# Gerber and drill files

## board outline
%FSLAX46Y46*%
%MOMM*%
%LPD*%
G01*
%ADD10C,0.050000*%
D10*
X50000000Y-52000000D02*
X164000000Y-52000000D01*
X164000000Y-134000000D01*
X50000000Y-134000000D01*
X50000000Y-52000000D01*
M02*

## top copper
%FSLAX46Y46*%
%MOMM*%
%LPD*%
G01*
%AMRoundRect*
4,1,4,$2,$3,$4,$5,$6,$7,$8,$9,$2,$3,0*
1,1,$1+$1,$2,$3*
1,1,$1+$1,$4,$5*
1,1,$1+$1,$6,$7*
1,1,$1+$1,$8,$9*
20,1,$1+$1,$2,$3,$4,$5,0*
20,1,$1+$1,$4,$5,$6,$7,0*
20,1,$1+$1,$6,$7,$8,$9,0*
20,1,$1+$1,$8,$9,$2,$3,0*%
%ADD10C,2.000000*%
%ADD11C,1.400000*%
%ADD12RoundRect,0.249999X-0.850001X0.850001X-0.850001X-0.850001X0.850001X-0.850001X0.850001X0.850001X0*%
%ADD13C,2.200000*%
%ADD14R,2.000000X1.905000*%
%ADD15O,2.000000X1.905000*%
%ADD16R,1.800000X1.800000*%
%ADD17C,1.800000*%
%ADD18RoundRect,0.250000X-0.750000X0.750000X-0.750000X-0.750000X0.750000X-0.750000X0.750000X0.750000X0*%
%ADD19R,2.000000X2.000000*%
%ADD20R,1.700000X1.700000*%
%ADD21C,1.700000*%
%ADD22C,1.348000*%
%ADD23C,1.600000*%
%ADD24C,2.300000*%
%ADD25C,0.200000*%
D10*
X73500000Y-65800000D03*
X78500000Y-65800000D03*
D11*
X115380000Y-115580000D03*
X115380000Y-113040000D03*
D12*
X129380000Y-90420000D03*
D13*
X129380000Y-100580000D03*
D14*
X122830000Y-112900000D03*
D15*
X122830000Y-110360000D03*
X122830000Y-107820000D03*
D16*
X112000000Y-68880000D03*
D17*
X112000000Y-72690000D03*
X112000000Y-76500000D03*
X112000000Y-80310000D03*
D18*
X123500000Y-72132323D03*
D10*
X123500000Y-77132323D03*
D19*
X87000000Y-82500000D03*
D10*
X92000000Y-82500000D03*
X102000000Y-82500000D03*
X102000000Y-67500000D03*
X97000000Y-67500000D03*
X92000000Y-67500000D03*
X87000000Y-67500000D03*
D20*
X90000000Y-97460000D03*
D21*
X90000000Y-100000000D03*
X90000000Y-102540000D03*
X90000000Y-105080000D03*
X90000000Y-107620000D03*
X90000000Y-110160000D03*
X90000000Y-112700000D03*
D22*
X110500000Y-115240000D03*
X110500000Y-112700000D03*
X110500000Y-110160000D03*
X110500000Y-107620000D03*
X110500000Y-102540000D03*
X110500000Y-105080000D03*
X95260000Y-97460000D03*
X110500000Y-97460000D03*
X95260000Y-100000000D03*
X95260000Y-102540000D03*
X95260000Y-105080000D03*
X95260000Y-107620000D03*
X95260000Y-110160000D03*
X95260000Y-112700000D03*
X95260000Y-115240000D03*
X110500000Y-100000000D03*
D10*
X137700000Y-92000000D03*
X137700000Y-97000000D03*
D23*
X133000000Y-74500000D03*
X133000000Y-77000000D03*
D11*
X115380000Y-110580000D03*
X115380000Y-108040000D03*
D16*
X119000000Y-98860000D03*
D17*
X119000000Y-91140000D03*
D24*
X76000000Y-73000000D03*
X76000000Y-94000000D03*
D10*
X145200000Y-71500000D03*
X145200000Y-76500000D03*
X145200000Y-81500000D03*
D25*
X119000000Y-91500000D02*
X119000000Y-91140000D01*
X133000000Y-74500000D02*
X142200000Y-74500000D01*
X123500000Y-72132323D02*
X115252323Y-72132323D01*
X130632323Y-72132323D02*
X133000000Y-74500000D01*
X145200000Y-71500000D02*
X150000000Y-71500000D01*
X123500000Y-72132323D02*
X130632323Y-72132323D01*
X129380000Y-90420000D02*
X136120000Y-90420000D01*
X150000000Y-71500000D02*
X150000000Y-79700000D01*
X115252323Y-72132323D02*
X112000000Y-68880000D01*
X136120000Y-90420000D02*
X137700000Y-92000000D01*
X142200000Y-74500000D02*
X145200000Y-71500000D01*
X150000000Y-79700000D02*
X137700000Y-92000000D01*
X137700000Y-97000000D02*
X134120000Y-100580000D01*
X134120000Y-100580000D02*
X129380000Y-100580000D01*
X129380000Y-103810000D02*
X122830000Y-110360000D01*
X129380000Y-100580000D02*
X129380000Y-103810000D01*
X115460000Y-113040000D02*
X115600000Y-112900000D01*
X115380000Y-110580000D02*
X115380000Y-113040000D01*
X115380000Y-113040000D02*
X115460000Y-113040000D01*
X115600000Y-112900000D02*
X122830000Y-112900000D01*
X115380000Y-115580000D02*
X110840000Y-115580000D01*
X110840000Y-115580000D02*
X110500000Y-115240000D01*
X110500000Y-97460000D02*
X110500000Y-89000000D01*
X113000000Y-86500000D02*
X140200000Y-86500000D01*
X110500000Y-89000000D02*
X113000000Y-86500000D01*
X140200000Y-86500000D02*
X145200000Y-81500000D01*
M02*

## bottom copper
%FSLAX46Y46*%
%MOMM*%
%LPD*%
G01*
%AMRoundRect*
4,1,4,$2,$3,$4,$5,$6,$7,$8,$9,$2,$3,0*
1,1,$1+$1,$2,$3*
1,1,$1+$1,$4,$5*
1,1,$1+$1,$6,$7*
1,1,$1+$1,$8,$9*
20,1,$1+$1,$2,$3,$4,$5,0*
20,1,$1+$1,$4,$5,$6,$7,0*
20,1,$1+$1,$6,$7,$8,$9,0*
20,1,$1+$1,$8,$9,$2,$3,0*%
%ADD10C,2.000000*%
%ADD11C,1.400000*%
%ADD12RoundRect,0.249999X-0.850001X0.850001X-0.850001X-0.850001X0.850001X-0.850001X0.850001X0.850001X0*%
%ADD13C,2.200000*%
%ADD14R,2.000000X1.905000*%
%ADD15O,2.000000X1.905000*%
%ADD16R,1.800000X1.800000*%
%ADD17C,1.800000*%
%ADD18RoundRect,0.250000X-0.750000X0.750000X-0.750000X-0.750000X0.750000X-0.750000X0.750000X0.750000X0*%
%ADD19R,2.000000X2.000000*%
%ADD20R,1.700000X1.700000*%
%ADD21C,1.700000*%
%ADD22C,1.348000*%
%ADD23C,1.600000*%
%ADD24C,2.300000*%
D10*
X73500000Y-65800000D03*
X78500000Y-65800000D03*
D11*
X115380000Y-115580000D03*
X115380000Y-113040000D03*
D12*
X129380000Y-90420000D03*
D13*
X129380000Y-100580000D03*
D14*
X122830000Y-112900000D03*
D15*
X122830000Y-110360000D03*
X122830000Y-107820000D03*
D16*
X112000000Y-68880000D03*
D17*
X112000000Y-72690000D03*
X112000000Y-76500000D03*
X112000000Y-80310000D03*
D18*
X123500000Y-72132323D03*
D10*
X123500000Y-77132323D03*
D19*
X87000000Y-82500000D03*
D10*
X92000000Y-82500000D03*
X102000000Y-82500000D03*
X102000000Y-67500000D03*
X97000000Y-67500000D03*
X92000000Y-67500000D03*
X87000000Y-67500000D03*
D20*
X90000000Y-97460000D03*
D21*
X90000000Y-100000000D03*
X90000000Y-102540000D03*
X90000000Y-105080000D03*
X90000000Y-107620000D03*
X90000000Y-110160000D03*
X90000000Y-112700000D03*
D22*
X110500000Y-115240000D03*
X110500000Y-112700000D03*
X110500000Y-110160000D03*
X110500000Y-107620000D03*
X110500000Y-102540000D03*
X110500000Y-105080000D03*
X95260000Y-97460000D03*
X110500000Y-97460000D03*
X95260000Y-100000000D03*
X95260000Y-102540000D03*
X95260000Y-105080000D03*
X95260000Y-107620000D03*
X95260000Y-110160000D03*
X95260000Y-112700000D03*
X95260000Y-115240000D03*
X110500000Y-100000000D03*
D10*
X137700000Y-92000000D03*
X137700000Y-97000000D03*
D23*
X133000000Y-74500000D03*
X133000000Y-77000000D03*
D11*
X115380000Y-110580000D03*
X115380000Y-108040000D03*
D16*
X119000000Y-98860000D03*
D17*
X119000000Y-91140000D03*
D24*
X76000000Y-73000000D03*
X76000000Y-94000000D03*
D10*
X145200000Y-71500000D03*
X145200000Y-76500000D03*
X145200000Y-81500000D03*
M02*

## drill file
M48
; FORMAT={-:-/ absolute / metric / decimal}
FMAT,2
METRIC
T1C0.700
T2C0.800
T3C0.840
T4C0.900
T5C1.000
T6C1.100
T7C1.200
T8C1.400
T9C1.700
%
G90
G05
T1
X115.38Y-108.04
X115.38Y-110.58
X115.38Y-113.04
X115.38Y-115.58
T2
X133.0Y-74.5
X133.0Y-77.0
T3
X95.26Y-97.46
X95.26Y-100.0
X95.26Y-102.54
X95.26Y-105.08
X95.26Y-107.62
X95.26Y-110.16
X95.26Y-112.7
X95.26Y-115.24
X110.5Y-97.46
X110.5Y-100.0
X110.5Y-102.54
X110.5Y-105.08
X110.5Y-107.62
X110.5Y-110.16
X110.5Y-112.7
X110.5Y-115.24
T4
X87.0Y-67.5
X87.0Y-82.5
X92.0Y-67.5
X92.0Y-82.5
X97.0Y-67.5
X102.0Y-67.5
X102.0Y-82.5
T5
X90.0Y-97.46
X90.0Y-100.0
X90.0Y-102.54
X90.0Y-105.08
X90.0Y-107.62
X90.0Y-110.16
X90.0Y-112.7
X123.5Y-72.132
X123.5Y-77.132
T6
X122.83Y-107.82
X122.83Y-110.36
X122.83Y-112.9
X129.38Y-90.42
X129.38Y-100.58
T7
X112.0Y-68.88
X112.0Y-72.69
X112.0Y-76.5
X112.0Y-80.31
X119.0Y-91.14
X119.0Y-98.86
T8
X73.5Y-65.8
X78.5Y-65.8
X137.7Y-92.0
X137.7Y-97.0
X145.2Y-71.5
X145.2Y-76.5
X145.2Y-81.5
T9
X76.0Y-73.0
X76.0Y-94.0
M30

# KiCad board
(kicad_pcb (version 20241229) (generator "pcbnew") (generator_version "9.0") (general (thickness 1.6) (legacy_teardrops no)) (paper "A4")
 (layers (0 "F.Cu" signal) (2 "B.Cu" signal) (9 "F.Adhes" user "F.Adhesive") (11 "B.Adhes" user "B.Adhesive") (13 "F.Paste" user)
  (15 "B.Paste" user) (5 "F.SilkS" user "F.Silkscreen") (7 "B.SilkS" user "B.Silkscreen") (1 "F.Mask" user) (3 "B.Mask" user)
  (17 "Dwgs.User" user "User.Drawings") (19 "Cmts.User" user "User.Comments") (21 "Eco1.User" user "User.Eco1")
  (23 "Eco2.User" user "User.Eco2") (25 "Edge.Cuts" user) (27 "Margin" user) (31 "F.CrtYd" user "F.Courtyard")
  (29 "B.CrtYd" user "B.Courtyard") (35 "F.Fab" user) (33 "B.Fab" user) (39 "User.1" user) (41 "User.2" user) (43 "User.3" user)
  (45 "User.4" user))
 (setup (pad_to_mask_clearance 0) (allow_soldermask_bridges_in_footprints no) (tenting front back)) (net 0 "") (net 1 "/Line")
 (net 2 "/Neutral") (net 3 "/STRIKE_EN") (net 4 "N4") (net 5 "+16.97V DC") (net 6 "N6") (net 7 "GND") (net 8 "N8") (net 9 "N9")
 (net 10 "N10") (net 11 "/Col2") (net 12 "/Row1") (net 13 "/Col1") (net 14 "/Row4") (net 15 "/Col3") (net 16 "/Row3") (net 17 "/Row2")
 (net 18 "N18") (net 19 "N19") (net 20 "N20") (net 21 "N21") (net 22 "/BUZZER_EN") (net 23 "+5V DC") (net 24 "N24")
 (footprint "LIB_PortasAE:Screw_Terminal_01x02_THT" (layer "F.Cu") (at 73.5 65.8)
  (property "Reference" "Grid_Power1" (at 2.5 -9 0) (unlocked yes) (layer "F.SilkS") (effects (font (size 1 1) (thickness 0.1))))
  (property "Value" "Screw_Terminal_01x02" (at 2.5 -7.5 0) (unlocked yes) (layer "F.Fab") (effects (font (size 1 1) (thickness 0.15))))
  (pad "1" thru_hole circle (at 0 0) (size 2 2) (drill 1.4) (layers "*.Cu" "*.Mask") (remove_unused_layers no) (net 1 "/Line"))
  (pad "2" thru_hole circle (at 5 0) (size 2 2) (drill 1.4) (layers "*.Cu" "*.Mask") (remove_unused_layers no) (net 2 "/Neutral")))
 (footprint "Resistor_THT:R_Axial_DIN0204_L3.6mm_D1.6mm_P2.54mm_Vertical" (layer "F.Cu") (at 115.38 115.58 90)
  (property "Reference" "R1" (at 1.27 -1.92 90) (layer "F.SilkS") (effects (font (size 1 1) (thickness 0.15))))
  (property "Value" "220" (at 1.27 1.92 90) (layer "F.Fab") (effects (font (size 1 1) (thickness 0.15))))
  (pad "1" thru_hole circle (at 0 0 90) (size 1.4 1.4) (drill 0.7) (layers "*.Cu" "*.Mask") (remove_unused_layers no) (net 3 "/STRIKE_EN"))
  (pad "2" thru_hole circle (at 2.54 0 90) (size 1.4 1.4) (drill 0.7) (layers "*.Cu" "*.Mask") (remove_unused_layers no) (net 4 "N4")))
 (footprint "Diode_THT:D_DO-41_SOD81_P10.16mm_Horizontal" (layer "F.Cu") (at 129.38 90.42 -90)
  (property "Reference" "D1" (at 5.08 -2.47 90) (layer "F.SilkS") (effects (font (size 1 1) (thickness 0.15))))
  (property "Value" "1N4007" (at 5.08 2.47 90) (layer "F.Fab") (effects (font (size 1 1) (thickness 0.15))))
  (pad "1" thru_hole roundrect (at 0 0 270) (size 2.2 2.2) (drill 1.1) (layers "*.Cu" "*.Mask") (remove_unused_layers no)
   (roundrect_rratio 0.113636) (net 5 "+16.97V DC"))
  (pad "2" thru_hole circle (at 10.16 0 270) (size 2.2 2.2) (drill 1.1) (layers "*.Cu" "*.Mask") (remove_unused_layers no) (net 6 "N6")))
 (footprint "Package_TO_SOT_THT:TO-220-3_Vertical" (layer "F.Cu") (at 122.83 112.9 90)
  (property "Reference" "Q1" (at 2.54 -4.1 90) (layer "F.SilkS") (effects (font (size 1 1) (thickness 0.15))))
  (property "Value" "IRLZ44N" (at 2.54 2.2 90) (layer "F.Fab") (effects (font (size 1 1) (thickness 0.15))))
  (pad "1" thru_hole rect (at 0 0 90) (size 1.905 2) (drill 1.1) (layers "*.Cu" "*.Mask") (remove_unused_layers no) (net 4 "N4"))
  (pad "2" thru_hole oval (at 2.54 0 90) (size 1.905 2) (drill 1.1) (layers "*.Cu" "*.Mask") (remove_unused_layers no) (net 6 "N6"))
  (pad "3" thru_hole oval (at 5.08 0 90) (size 1.905 2) (drill 1.1) (layers "*.Cu" "*.Mask") (remove_unused_layers no) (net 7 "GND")))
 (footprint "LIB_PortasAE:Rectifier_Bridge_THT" (layer "F.Cu") (at 112 68.88 -90)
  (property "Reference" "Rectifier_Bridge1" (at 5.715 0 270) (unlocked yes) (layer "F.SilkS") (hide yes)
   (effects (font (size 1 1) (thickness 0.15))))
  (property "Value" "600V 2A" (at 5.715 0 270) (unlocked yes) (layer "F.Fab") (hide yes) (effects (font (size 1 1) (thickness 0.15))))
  (pad "1" thru_hole rect (at 0 0 270) (size 1.8 1.8) (drill 1.2) (layers "*.Cu" "*.Mask") (remove_unused_layers no) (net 5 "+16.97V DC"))
  (pad "2" thru_hole circle (at 3.81 0 270) (size 1.8 1.8) (drill 1.2) (layers "*.Cu" "*.Mask") (remove_unused_layers no) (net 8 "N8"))
  (pad "3" thru_hole circle (at 7.62 0 270) (size 1.8 1.8) (drill 1.2) (layers "*.Cu" "*.Mask") (remove_unused_layers no) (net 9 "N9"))
  (pad "4" thru_hole circle (at 11.43 0 270) (size 1.8 1.8) (drill 1.2) (layers "*.Cu" "*.Mask") (remove_unused_layers no) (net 7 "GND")))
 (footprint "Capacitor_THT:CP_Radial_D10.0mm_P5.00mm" (layer "F.Cu") (at 123.5 72.132323 -90)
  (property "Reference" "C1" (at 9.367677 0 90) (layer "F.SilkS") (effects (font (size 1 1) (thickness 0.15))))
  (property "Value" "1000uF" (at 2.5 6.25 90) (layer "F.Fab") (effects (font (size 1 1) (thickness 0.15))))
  (pad "1" thru_hole roundrect (at 0 0 270) (size 2 2) (drill 1) (layers "*.Cu" "*.Mask") (remove_unused_layers no) (roundrect_rratio 0.125)
   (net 5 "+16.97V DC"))
  (pad "2" thru_hole circle (at 5 0 270) (size 2 2) (drill 1) (layers "*.Cu" "*.Mask") (remove_unused_layers no) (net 7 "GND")))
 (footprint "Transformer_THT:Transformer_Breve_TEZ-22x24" (layer "F.Cu") (at 87 82.5)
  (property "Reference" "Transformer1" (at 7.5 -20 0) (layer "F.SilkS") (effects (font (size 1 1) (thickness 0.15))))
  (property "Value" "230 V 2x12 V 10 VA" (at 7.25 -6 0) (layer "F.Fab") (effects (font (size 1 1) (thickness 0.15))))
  (pad "1" thru_hole rect (at 0 0) (size 2 2) (drill 0.9) (layers "*.Cu" "*.Mask") (remove_unused_layers no) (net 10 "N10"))
  (pad "2" thru_hole circle (at 5 0) (size 2 2) (drill 0.9) (layers "*.Cu" "*.Mask") (remove_unused_layers no))
  (pad "4" thru_hole circle (at 15 0) (size 2 2) (drill 0.9) (layers "*.Cu" "*.Mask") (remove_unused_layers no) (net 2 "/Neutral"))
  (pad "5" thru_hole circle (at 15 -15) (size 2 2) (drill 0.9) (layers "*.Cu" "*.Mask") (remove_unused_layers no) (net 8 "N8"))
  (pad "6" thru_hole circle (at 10 -15) (size 2 2) (drill 0.9) (layers "*.Cu" "*.Mask") (remove_unused_layers no) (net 9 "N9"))
  (pad "7" thru_hole circle (at 5 -15) (size 2 2) (drill 0.9) (layers "*.Cu" "*.Mask") (remove_unused_layers no) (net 8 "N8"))
  (pad "8" thru_hole circle (at 0 -15) (size 2 2) (drill 0.9) (layers "*.Cu" "*.Mask") (remove_unused_layers no) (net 9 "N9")))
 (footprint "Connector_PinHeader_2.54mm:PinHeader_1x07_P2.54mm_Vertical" (layer "F.Cu") (at 90 97.46)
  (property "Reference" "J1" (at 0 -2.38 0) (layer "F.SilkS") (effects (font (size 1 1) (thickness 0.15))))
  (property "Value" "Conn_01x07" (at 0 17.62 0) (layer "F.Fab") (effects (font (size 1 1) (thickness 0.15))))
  (pad "1" thru_hole rect (at 0 0) (size 1.7 1.7) (drill 1) (layers "*.Cu" "*.Mask") (remove_unused_layers no) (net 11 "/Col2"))
  (pad "2" thru_hole circle (at 0 2.54) (size 1.7 1.7) (drill 1) (layers "*.Cu" "*.Mask") (remove_unused_layers no) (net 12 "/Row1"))
  (pad "3" thru_hole circle (at 0 5.08) (size 1.7 1.7) (drill 1) (layers "*.Cu" "*.Mask") (remove_unused_layers no) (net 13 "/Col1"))
  (pad "4" thru_hole circle (at 0 7.62) (size 1.7 1.7) (drill 1) (layers "*.Cu" "*.Mask") (remove_unused_layers no) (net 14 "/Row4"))
  (pad "5" thru_hole circle (at 0 10.16) (size 1.7 1.7) (drill 1) (layers "*.Cu" "*.Mask") (remove_unused_layers no) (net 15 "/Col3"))
  (pad "6" thru_hole circle (at 0 12.7) (size 1.7 1.7) (drill 1) (layers "*.Cu" "*.Mask") (remove_unused_layers no) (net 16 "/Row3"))
  (pad "7" thru_hole circle (at 0 15.24) (size 1.7 1.7) (drill 1) (layers "*.Cu" "*.Mask") (remove_unused_layers no) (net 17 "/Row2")))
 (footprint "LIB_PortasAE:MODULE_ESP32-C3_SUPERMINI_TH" (layer "F.Cu") (at 102.88 107.36)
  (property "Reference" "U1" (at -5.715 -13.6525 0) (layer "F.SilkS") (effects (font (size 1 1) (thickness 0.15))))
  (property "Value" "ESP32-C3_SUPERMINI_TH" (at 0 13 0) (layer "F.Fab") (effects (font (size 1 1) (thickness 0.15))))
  (pad "0" thru_hole circle (at 7.62 7.88) (size 1.348 1.348) (drill 0.84) (layers "*.Cu" "*.Mask") (remove_unused_layers no)
   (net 3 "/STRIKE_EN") (solder_mask_margin 0.102))
  (pad "1" thru_hole circle (at 7.62 5.34) (size 1.348 1.348) (drill 0.84) (layers "*.Cu" "*.Mask") (remove_unused_layers no) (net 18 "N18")
   (solder_mask_margin 0.102))
  (pad "2" thru_hole circle (at 7.62 2.8) (size 1.348 1.348) (drill 0.84) (layers "*.Cu" "*.Mask") (remove_unused_layers no) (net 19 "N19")
   (solder_mask_margin 0.102))
  (pad "3" thru_hole circle (at 7.62 0.26) (size 1.348 1.348) (drill 0.84) (layers "*.Cu" "*.Mask") (remove_unused_layers no) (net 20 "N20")
   (solder_mask_margin 0.102))
  (pad "3.3" thru_hole circle (at 7.62 -4.82) (size 1.348 1.348) (drill 0.84) (layers "*.Cu" "*.Mask") (remove_unused_layers no)
   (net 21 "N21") (solder_mask_margin 0.102))
  (pad "4" thru_hole circle (at 7.62 -2.28) (size 1.348 1.348) (drill 0.84) (layers "*.Cu" "*.Mask") (remove_unused_layers no)
   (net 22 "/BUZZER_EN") (solder_mask_margin 0.102))
  (pad "5" thru_hole circle (at -7.62 -9.9) (size 1.348 1.348) (drill 0.84) (layers "*.Cu" "*.Mask") (remove_unused_layers no)
   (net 11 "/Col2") (solder_mask_margin 0.102))
  (pad "5V" thru_hole circle (at 7.62 -9.9) (size 1.348 1.348) (drill 0.84) (layers "*.Cu" "*.Mask") (remove_unused_layers no)
   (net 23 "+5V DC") (solder_mask_margin 0.102))
  (pad "6" thru_hole circle (at -7.62 -7.36) (size 1.348 1.348) (drill 0.84) (layers "*.Cu" "*.Mask") (remove_unused_layers no)
   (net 12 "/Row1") (solder_mask_margin 0.102))
  (pad "7" thru_hole circle (at -7.62 -4.82) (size 1.348 1.348) (drill 0.84) (layers "*.Cu" "*.Mask") (remove_unused_layers no)
   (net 13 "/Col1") (solder_mask_margin 0.102))
  (pad "8" thru_hole circle (at -7.62 -2.28) (size 1.348 1.348) (drill 0.84) (layers "*.Cu" "*.Mask") (remove_unused_layers no)
   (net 14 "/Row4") (solder_mask_margin 0.102))
  (pad "9" thru_hole circle (at -7.62 0.26) (size 1.348 1.348) (drill 0.84) (layers "*.Cu" "*.Mask") (remove_unused_layers no)
   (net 15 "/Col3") (solder_mask_margin 0.102))
  (pad "10" thru_hole circle (at -7.62 2.8) (size 1.348 1.348) (drill 0.84) (layers "*.Cu" "*.Mask") (remove_unused_layers no)
   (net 16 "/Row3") (solder_mask_margin 0.102))
  (pad "20" thru_hole circle (at -7.62 5.34) (size 1.348 1.348) (drill 0.84) (layers "*.Cu" "*.Mask") (remove_unused_layers no)
   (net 17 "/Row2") (solder_mask_margin 0.102))
  (pad "21" thru_hole circle (at -7.62 7.88) (size 1.348 1.348) (drill 0.84) (layers "*.Cu" "*.Mask") (remove_unused_layers no)
   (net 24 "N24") (solder_mask_margin 0.102))
  (pad "G" thru_hole circle (at 7.62 -7.36) (size 1.348 1.348) (drill 0.84) (layers "*.Cu" "*.Mask") (remove_unused_layers no) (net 7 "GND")
   (solder_mask_margin 0.102)))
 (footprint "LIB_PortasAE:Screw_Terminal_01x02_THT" (layer "F.Cu") (at 137.7 92 -90)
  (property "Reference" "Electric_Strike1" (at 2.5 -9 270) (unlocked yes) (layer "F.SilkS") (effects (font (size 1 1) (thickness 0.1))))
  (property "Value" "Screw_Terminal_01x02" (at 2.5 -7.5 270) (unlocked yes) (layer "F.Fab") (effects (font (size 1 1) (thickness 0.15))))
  (pad "1" thru_hole circle (at 0 0 270) (size 2 2) (drill 1.4) (layers "*.Cu" "*.Mask") (remove_unused_layers no) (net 5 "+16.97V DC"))
  (pad "2" thru_hole circle (at 5 0 270) (size 2 2) (drill 1.4) (layers "*.Cu" "*.Mask") (remove_unused_layers no) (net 6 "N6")))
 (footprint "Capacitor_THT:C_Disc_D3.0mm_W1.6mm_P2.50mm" (layer "F.Cu") (at 133 74.5 -90)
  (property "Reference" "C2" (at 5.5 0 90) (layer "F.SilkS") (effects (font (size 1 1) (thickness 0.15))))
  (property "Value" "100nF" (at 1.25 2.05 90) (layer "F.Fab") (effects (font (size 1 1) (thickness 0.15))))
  (pad "1" thru_hole circle (at 0 0 270) (size 1.6 1.6) (drill 0.8) (layers "*.Cu" "*.Mask") (remove_unused_layers no) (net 5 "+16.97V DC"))
  (pad "2" thru_hole circle (at 2.5 0 270) (size 1.6 1.6) (drill 0.8) (layers "*.Cu" "*.Mask") (remove_unused_layers no) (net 7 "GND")))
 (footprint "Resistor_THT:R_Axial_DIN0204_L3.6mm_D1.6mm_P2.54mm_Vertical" (layer "F.Cu") (at 115.38 110.58 90)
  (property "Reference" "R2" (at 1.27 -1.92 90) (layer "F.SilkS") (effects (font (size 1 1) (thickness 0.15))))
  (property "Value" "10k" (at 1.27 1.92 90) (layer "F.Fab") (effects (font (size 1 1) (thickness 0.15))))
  (pad "1" thru_hole circle (at 0 0 90) (size 1.4 1.4) (drill 0.7) (layers "*.Cu" "*.Mask") (remove_unused_layers no) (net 4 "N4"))
  (pad "2" thru_hole circle (at 2.54 0 90) (size 1.4 1.4) (drill 0.7) (layers "*.Cu" "*.Mask") (remove_unused_layers no) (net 7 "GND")))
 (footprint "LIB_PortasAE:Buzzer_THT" (layer "F.Cu") (at 119 98.86 90)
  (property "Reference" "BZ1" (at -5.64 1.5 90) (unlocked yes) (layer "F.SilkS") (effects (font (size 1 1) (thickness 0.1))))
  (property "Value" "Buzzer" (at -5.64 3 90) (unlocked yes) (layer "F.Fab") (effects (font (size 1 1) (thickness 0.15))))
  (pad "1" thru_hole rect (at 0 0 90) (size 1.8 1.8) (drill 1.2) (layers "*.Cu" "*.Mask") (remove_unused_layers no) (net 22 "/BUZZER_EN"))
  (pad "2" thru_hole circle (at 7.72 0 90) (size 1.8 1.8) (drill 1.2) (layers "*.Cu" "*.Mask") (remove_unused_layers no) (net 7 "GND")))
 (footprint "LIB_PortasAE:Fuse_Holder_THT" (layer "F.Cu") (at 76 73 -90)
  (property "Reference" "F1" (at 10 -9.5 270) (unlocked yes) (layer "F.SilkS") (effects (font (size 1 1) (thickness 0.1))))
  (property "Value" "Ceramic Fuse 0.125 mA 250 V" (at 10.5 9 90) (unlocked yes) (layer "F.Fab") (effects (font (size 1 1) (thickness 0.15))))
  (pad "1" thru_hole circle (at 0 0 270) (size 2.3 2.3) (drill 1.7) (layers "*.Cu" "*.Mask") (remove_unused_layers no) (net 1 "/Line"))
  (pad "2" thru_hole circle (at 21 0 270) (size 2.3 2.3) (drill 1.7) (layers "*.Cu" "*.Mask") (remove_unused_layers no) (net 10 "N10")))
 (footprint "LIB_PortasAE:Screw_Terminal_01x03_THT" (layer "F.Cu") (at 145.2 71.5 -90)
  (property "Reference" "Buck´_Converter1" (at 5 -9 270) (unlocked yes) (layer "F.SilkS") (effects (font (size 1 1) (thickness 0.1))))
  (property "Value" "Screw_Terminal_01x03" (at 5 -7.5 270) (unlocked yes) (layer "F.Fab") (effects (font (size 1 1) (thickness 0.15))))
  (pad "1" thru_hole circle (at 0 0 270) (size 2 2) (drill 1.4) (layers "*.Cu" "*.Mask") (remove_unused_layers no) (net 5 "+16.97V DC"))
  (pad "2" thru_hole circle (at 5 0 270) (size 2 2) (drill 1.4) (layers "*.Cu" "*.Mask") (remove_unused_layers no) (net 7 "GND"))
  (pad "3" thru_hole circle (at 10 0 270) (size 2 2) (drill 1.4) (layers "*.Cu" "*.Mask") (remove_unused_layers no) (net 23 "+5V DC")))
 (gr_rect (start 50 52) (end 164 134) (stroke (width 0.05) (type default)) (fill no) (layer "Edge.Cuts"))
 (segment (start 119 91.5) (end 119 91.14) (width 0.2) (layer "F.Cu") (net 7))
 (segment (start 133 74.5) (end 142.2 74.5) (width 0.2) (layer "F.Cu") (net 5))
 (segment (start 123.5 72.132323) (end 115.252323 72.132323) (width 0.2) (layer "F.Cu") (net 5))
 (segment (start 130.632323 72.132323) (end 133 74.5) (width 0.2) (layer "F.Cu") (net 5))
 (segment (start 145.2 71.5) (end 150 71.5) (width 0.2) (layer "F.Cu") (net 5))
 (segment (start 123.5 72.132323) (end 130.632323 72.132323) (width 0.2) (layer "F.Cu") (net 5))
 (segment (start 129.38 90.42) (end 136.12 90.42) (width 0.2) (layer "F.Cu") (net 5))
 (segment (start 150 71.5) (end 150 79.7) (width 0.2) (layer "F.Cu") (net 5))
 (segment (start 115.252323 72.132323) (end 112 68.88) (width 0.2) (layer "F.Cu") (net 5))
 (segment (start 136.12 90.42) (end 137.7 92) (width 0.2) (layer "F.Cu") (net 5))
 (segment (start 142.2 74.5) (end 145.2 71.5) (width 0.2) (layer "F.Cu") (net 5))
 (segment (start 150 79.7) (end 137.7 92) (width 0.2) (layer "F.Cu") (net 5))
 (segment (start 137.7 97) (end 134.12 100.58) (width 0.2) (layer "F.Cu") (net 6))
 (segment (start 134.12 100.58) (end 129.38 100.58) (width 0.2) (layer "F.Cu") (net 6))
 (segment (start 129.38 103.81) (end 122.83 110.36) (width 0.2) (layer "F.Cu") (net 6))
 (segment (start 129.38 100.58) (end 129.38 103.81) (width 0.2) (layer "F.Cu") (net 6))
 (segment (start 115.46 113.04) (end 115.6 112.9) (width 0.2) (layer "F.Cu") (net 4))
 (segment (start 115.38 110.58) (end 115.38 113.04) (width 0.2) (layer "F.Cu") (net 4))
 (segment (start 115.38 113.04) (end 115.46 113.04) (width 0.2) (layer "F.Cu") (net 4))
 (segment (start 115.6 112.9) (end 122.83 112.9) (width 0.2) (layer "F.Cu") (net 4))
 (segment (start 115.38 115.58) (end 110.84 115.58) (width 0.2) (layer "F.Cu") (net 3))
 (segment (start 110.84 115.58) (end 110.5 115.24) (width 0.2) (layer "F.Cu") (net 3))
 (segment (start 110.5 97.46) (end 110.5 89) (width 0.2) (layer "F.Cu") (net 23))
 (segment (start 113 86.5) (end 140.2 86.5) (width 0.2) (layer "F.Cu") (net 23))
 (segment (start 110.5 89) (end 113 86.5) (width 0.2) (layer "F.Cu") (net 23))
 (segment (start 140.2 86.5) (end 145.2 81.5) (width 0.2) (layer "F.Cu") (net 23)))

